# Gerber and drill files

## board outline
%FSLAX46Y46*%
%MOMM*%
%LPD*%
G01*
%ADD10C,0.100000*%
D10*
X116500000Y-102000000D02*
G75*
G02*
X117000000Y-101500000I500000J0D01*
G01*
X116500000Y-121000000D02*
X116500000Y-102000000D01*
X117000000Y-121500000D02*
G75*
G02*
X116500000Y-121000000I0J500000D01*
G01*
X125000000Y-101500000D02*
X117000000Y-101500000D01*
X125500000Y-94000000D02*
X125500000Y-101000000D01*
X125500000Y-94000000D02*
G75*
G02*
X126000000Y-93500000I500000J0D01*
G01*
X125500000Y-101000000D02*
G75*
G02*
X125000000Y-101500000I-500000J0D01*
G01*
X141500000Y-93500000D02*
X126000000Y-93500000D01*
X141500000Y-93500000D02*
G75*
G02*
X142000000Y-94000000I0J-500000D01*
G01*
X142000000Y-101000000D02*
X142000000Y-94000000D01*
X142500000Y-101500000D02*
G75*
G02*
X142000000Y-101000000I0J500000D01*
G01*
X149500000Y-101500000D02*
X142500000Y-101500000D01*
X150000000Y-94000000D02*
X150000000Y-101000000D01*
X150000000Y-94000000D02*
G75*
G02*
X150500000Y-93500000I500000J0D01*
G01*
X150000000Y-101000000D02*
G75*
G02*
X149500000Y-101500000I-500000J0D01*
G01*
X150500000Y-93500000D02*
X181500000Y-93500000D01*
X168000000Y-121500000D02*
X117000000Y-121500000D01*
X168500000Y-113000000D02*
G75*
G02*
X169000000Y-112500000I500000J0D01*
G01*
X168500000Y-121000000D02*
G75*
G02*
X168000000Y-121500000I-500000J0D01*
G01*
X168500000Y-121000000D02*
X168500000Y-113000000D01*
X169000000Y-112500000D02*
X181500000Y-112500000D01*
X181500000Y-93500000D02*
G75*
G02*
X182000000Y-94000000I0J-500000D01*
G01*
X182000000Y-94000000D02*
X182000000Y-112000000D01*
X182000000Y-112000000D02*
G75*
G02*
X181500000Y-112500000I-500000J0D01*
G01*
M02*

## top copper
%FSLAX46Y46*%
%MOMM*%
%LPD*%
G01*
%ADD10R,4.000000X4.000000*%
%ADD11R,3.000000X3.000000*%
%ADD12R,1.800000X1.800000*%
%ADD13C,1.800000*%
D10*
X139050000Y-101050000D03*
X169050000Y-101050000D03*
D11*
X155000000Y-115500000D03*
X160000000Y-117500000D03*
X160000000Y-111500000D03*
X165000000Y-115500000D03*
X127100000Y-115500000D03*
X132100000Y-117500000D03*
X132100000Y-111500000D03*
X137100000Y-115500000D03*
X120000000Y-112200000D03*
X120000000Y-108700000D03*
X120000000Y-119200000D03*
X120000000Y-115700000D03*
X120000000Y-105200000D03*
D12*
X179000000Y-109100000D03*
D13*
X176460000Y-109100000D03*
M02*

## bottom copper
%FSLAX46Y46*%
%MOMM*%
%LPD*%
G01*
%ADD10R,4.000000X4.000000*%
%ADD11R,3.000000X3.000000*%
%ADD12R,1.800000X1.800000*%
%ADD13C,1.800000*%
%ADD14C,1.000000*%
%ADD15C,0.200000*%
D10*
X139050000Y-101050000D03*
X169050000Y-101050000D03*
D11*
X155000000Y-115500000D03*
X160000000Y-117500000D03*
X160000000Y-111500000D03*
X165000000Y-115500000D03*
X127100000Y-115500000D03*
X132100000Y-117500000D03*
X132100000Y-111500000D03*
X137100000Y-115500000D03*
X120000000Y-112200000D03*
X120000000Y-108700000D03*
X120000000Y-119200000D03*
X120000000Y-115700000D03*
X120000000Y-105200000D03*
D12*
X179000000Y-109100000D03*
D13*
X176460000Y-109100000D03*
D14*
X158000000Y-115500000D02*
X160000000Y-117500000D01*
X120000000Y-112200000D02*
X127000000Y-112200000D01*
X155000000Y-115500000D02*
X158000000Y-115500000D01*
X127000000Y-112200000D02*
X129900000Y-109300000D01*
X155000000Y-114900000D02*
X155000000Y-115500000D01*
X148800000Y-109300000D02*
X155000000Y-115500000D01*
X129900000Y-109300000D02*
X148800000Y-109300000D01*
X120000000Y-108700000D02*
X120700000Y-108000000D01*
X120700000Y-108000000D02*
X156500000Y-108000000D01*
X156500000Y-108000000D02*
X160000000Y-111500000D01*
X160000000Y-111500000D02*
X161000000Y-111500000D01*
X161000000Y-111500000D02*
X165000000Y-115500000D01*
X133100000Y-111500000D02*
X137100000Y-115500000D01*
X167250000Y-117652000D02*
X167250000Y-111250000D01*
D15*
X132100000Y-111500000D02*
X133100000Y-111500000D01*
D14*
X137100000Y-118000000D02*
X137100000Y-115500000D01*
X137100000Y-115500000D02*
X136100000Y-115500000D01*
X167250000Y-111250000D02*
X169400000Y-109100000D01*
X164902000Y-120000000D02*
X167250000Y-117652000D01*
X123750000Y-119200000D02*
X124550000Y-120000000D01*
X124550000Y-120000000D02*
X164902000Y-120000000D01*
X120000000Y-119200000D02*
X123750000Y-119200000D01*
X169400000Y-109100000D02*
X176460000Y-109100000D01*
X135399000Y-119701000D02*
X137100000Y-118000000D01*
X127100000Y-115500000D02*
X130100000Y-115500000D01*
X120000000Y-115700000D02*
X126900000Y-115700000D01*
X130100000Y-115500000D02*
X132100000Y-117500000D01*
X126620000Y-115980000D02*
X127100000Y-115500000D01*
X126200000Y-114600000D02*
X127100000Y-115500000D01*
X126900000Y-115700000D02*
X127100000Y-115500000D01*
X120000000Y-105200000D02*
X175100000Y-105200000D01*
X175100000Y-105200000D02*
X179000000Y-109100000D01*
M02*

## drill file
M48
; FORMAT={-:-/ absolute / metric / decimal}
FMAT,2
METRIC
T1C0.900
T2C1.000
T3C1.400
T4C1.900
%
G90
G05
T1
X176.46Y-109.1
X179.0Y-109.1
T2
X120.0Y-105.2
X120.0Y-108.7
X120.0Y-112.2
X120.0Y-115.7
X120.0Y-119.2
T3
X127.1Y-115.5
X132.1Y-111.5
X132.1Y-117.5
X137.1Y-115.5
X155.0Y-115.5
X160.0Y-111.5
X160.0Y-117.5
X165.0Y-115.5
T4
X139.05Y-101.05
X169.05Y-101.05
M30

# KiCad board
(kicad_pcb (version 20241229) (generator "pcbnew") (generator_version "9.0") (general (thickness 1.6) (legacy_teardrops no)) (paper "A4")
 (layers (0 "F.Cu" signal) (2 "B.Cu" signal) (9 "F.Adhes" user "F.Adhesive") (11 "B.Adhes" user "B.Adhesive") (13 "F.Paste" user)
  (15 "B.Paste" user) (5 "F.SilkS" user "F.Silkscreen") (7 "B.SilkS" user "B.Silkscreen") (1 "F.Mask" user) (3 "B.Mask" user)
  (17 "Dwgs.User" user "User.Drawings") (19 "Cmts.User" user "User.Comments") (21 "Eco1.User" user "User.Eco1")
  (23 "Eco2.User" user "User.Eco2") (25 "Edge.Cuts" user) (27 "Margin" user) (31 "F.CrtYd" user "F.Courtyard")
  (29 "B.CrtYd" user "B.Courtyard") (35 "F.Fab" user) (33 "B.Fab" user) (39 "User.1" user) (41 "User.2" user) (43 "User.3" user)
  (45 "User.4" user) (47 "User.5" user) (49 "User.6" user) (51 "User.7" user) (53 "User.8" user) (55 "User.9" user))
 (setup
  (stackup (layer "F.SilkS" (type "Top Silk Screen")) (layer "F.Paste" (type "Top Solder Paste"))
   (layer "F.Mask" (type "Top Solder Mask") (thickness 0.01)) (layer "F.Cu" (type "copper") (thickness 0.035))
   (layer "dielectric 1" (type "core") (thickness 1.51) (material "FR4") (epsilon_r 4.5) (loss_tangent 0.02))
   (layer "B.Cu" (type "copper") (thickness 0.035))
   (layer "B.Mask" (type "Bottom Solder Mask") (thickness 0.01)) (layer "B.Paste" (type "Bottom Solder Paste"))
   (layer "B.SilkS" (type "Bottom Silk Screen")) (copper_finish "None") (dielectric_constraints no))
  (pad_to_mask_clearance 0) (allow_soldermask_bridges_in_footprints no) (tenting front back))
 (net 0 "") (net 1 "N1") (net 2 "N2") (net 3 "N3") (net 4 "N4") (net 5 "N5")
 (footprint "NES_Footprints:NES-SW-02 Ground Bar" (layer "F.Cu") (at 154.05 101.05)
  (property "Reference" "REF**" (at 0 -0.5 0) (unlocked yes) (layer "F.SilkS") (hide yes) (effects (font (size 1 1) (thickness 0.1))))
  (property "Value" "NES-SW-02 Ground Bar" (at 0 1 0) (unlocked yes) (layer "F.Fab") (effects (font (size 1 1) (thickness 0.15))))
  (pad "1" thru_hole rect (at -15 0) (size 4 4) (drill 1.9) (layers "*.Cu" "B.Mask") (remove_unused_layers no))
  (pad "1" thru_hole rect (at 15 0) (size 4 4) (drill 1.9) (layers "*.Cu" "B.Mask") (remove_unused_layers no)))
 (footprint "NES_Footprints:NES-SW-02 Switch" (layer "F.Cu") (at 160 115.5)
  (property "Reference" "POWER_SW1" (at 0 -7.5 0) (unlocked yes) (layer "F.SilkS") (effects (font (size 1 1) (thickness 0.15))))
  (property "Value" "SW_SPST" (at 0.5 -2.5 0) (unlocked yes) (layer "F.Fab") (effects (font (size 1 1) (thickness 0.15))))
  (pad "1" thru_hole rect (at -5 0 180) (size 3 3) (drill 1.4) (layers "*.Cu" "B.Mask") (remove_unused_layers no) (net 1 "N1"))
  (pad "1" thru_hole rect (at 0 2 180) (size 3 3) (drill 1.4) (layers "*.Cu" "B.Mask") (remove_unused_layers no) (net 1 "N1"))
  (pad "2" thru_hole rect (at 0 -4 180) (size 3 3) (drill 1.4) (layers "*.Cu" "B.Mask") (remove_unused_layers no) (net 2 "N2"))
  (pad "2" thru_hole rect (at 5 0 180) (size 3 3) (drill 1.4) (layers "*.Cu" "B.Mask") (remove_unused_layers no) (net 2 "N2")))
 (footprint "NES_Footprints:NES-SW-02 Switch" (layer "F.Cu") (at 132.1 115.5)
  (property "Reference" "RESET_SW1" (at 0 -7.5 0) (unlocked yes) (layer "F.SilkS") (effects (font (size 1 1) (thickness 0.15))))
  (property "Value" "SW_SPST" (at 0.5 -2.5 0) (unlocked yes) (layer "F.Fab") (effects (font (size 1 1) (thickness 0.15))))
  (pad "1" thru_hole rect (at -5 0 180) (size 3 3) (drill 1.4) (layers "*.Cu" "B.Mask") (remove_unused_layers no) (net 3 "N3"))
  (pad "1" thru_hole rect (at 0 2 180) (size 3 3) (drill 1.4) (layers "*.Cu" "B.Mask") (remove_unused_layers no) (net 3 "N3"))
  (pad "2" thru_hole rect (at 0 -4 180) (size 3 3) (drill 1.4) (layers "*.Cu" "B.Mask") (remove_unused_layers no) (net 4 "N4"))
  (pad "2" thru_hole rect (at 5 0 180) (size 3 3) (drill 1.4) (layers "*.Cu" "B.Mask") (remove_unused_layers no) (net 4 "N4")))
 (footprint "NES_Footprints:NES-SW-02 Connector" (layer "F.Cu") (at 120 112.2 90)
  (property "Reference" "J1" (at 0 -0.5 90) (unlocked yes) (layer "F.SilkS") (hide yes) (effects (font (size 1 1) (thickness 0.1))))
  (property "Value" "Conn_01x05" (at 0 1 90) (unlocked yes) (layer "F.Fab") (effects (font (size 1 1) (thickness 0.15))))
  (pad "1" thru_hole rect (at 0 0 90) (size 3 3) (drill 1) (layers "*.Cu" "B.Mask") (remove_unused_layers no) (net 1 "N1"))
  (pad "2" thru_hole rect (at 3.5 0 90) (size 3 3) (drill 1) (layers "*.Cu" "B.Mask") (remove_unused_layers no) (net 2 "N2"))
  (pad "3" thru_hole rect (at -7 0 90) (size 3 3) (drill 1) (layers "*.Cu" "B.Mask") (remove_unused_layers no) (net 4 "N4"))
  (pad "4" thru_hole rect (at -3.5 0 90) (size 3 3) (drill 1) (layers "*.Cu" "B.Mask") (remove_unused_layers no) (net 3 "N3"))
  (pad "5" thru_hole rect (at 7 0 90) (size 3 3) (drill 1) (layers "*.Cu" "B.Mask") (remove_unused_layers no) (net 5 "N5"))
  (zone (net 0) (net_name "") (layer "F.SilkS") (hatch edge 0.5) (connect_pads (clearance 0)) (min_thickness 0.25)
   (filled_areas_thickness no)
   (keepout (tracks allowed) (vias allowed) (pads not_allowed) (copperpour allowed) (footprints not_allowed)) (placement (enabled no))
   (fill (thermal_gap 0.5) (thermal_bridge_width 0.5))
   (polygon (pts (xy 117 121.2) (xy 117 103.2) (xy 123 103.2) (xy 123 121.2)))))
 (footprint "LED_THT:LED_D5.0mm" (layer "F.Cu") (at 179 109.1 180)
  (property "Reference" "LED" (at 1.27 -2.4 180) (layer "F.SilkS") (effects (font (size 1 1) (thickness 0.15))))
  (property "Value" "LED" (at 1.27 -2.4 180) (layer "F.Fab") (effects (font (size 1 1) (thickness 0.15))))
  (pad "1" thru_hole rect (at 0 0 180) (size 1.8 1.8) (drill 0.9) (layers "*.Cu" "B.Mask") (remove_unused_layers no) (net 5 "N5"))
  (pad "2" thru_hole circle (at 2.54 0 180) (size 1.8 1.8) (drill 0.9) (layers "*.Cu" "B.Mask") (remove_unused_layers no) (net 4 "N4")))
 (gr_arc (start 116.5 102) (mid 116.646447 101.646447) (end 117 101.5) (stroke (width 0.1) (type solid)) (layer "Edge.Cuts"))
 (gr_line (start 116.5 121) (end 116.5 102) (stroke (width 0.1) (type solid)) (layer "Edge.Cuts"))
 (gr_arc (start 117 121.5) (mid 116.646447 121.353553) (end 116.5 121) (stroke (width 0.1) (type solid)) (layer "Edge.Cuts"))
 (gr_line (start 125 101.5) (end 117 101.5) (stroke (width 0.1) (type solid)) (layer "Edge.Cuts"))
 (gr_line (start 125.5 94) (end 125.5 101) (stroke (width 0.1) (type solid)) (layer "Edge.Cuts"))
 (gr_arc (start 125.5 94) (mid 125.646447 93.646447) (end 126 93.5) (stroke (width 0.1) (type solid)) (layer "Edge.Cuts"))
 (gr_arc (start 125.5 101) (mid 125.353553 101.353553) (end 125 101.5) (stroke (width 0.1) (type solid)) (layer "Edge.Cuts"))
 (gr_line (start 141.5 93.5) (end 126 93.5) (stroke (width 0.1) (type solid)) (layer "Edge.Cuts"))
 (gr_arc (start 141.5 93.5) (mid 141.853553 93.646447) (end 142 94) (stroke (width 0.1) (type solid)) (layer "Edge.Cuts"))
 (gr_line (start 142 101) (end 142 94) (stroke (width 0.1) (type solid)) (layer "Edge.Cuts"))
 (gr_arc (start 142.5 101.5) (mid 142.146447 101.353553) (end 142 101) (stroke (width 0.1) (type solid)) (layer "Edge.Cuts"))
 (gr_line (start 149.5 101.5) (end 142.5 101.5) (stroke (width 0.1) (type solid)) (layer "Edge.Cuts"))
 (gr_line (start 150 94) (end 150 101) (stroke (width 0.1) (type solid)) (layer "Edge.Cuts"))
 (gr_arc (start 150 94) (mid 150.146447 93.646447) (end 150.5 93.5) (stroke (width 0.1) (type solid)) (layer "Edge.Cuts"))
 (gr_arc (start 150 101) (mid 149.853553 101.353553) (end 149.5 101.5) (stroke (width 0.1) (type solid)) (layer "Edge.Cuts"))
 (gr_line (start 150.5 93.5) (end 181.5 93.5) (stroke (width 0.1) (type solid)) (layer "Edge.Cuts"))
 (gr_line (start 168 121.5) (end 117 121.5) (stroke (width 0.1) (type solid)) (layer "Edge.Cuts"))
 (gr_arc (start 168.5 113) (mid 168.646447 112.646447) (end 169 112.5) (stroke (width 0.1) (type solid)) (layer "Edge.Cuts"))
 (gr_arc (start 168.5 121) (mid 168.353553 121.353553) (end 168 121.5) (stroke (width 0.1) (type solid)) (layer "Edge.Cuts"))
 (gr_line (start 168.5 121) (end 168.5 113) (stroke (width 0.1) (type solid)) (layer "Edge.Cuts"))
 (gr_line (start 169 112.5) (end 181.5 112.5) (stroke (width 0.1) (type solid)) (layer "Edge.Cuts"))
 (gr_arc (start 181.5 93.5) (mid 181.853553 93.646447) (end 182 94) (stroke (width 0.1) (type solid)) (layer "Edge.Cuts"))
 (gr_line (start 182 94) (end 182 112) (stroke (width 0.1) (type solid)) (layer "Edge.Cuts"))
 (gr_arc (start 182 112) (mid 181.853553 112.353553) (end 181.5 112.5) (stroke (width 0.1) (type solid)) (layer "Edge.Cuts"))
 (segment (start 158 115.5) (end 160 117.5) (width 1) (layer "B.Cu") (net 1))
 (segment (start 120 112.2) (end 127 112.2) (width 1) (layer "B.Cu") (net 1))
 (segment (start 155 115.5) (end 158 115.5) (width 1) (layer "B.Cu") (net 1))
 (segment (start 127 112.2) (end 129.9 109.3) (width 1) (layer "B.Cu") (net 1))
 (segment (start 155 114.9) (end 155 115.5) (width 1) (layer "B.Cu") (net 1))
 (segment (start 148.8 109.3) (end 155 115.5) (width 1) (layer "B.Cu") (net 1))
 (segment (start 129.9 109.3) (end 148.8 109.3) (width 1) (layer "B.Cu") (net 1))
 (segment (start 120 108.7) (end 120.7 108) (width 1) (layer "B.Cu") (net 2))
 (segment (start 120.7 108) (end 156.5 108) (width 1) (layer "B.Cu") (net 2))
 (segment (start 156.5 108) (end 160 111.5) (width 1) (layer "B.Cu") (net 2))
 (segment (start 160 111.5) (end 161 111.5) (width 1) (layer "B.Cu") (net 2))
 (segment (start 161 111.5) (end 165 115.5) (width 1) (layer "B.Cu") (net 2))
 (segment (start 133.1 111.5) (end 137.1 115.5) (width 1) (layer "B.Cu") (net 4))
 (segment (start 167.25 117.652) (end 167.25 111.25) (width 1) (layer "B.Cu") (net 4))
 (segment (start 132.1 111.5) (end 133.1 111.5) (width 0.2) (layer "B.Cu") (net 4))
 (segment (start 137.1 118) (end 137.1 115.5) (width 1) (layer "B.Cu") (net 4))
 (segment (start 137.1 115.5) (end 136.1 115.5) (width 1) (layer "B.Cu") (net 4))
 (segment (start 167.25 111.25) (end 169.4 109.1) (width 1) (layer "B.Cu") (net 4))
 (segment (start 164.902 120) (end 167.25 117.652) (width 1) (layer "B.Cu") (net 4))
 (segment (start 123.75 119.2) (end 124.55 120) (width 1) (layer "B.Cu") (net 4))
 (segment (start 124.55 120) (end 164.902 120) (width 1) (layer "B.Cu") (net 4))
 (segment (start 120 119.2) (end 123.75 119.2) (width 1) (layer "B.Cu") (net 4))
 (segment (start 169.4 109.1) (end 176.46 109.1) (width 1) (layer "B.Cu") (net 4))
 (segment (start 135.399 119.701) (end 137.1 118) (width 1) (layer "B.Cu") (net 4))
 (segment (start 127.1 115.5) (end 130.1 115.5) (width 1) (layer "B.Cu") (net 3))
 (segment (start 120 115.7) (end 126.9 115.7) (width 1) (layer "B.Cu") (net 3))
 (segment (start 130.1 115.5) (end 132.1 117.5) (width 1) (layer "B.Cu") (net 3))
 (segment (start 126.62 115.98) (end 127.1 115.5) (width 1) (layer "B.Cu") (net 3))
 (segment (start 126.2 114.6) (end 127.1 115.5) (width 1) (layer "B.Cu") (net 3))
 (segment (start 126.9 115.7) (end 127.1 115.5) (width 1) (layer "B.Cu") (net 3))
 (segment (start 120 105.2) (end 175.1 105.2) (width 1) (layer "B.Cu") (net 5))
 (segment (start 175.1 105.2) (end 179 109.1) (width 1) (layer "B.Cu") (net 5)))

